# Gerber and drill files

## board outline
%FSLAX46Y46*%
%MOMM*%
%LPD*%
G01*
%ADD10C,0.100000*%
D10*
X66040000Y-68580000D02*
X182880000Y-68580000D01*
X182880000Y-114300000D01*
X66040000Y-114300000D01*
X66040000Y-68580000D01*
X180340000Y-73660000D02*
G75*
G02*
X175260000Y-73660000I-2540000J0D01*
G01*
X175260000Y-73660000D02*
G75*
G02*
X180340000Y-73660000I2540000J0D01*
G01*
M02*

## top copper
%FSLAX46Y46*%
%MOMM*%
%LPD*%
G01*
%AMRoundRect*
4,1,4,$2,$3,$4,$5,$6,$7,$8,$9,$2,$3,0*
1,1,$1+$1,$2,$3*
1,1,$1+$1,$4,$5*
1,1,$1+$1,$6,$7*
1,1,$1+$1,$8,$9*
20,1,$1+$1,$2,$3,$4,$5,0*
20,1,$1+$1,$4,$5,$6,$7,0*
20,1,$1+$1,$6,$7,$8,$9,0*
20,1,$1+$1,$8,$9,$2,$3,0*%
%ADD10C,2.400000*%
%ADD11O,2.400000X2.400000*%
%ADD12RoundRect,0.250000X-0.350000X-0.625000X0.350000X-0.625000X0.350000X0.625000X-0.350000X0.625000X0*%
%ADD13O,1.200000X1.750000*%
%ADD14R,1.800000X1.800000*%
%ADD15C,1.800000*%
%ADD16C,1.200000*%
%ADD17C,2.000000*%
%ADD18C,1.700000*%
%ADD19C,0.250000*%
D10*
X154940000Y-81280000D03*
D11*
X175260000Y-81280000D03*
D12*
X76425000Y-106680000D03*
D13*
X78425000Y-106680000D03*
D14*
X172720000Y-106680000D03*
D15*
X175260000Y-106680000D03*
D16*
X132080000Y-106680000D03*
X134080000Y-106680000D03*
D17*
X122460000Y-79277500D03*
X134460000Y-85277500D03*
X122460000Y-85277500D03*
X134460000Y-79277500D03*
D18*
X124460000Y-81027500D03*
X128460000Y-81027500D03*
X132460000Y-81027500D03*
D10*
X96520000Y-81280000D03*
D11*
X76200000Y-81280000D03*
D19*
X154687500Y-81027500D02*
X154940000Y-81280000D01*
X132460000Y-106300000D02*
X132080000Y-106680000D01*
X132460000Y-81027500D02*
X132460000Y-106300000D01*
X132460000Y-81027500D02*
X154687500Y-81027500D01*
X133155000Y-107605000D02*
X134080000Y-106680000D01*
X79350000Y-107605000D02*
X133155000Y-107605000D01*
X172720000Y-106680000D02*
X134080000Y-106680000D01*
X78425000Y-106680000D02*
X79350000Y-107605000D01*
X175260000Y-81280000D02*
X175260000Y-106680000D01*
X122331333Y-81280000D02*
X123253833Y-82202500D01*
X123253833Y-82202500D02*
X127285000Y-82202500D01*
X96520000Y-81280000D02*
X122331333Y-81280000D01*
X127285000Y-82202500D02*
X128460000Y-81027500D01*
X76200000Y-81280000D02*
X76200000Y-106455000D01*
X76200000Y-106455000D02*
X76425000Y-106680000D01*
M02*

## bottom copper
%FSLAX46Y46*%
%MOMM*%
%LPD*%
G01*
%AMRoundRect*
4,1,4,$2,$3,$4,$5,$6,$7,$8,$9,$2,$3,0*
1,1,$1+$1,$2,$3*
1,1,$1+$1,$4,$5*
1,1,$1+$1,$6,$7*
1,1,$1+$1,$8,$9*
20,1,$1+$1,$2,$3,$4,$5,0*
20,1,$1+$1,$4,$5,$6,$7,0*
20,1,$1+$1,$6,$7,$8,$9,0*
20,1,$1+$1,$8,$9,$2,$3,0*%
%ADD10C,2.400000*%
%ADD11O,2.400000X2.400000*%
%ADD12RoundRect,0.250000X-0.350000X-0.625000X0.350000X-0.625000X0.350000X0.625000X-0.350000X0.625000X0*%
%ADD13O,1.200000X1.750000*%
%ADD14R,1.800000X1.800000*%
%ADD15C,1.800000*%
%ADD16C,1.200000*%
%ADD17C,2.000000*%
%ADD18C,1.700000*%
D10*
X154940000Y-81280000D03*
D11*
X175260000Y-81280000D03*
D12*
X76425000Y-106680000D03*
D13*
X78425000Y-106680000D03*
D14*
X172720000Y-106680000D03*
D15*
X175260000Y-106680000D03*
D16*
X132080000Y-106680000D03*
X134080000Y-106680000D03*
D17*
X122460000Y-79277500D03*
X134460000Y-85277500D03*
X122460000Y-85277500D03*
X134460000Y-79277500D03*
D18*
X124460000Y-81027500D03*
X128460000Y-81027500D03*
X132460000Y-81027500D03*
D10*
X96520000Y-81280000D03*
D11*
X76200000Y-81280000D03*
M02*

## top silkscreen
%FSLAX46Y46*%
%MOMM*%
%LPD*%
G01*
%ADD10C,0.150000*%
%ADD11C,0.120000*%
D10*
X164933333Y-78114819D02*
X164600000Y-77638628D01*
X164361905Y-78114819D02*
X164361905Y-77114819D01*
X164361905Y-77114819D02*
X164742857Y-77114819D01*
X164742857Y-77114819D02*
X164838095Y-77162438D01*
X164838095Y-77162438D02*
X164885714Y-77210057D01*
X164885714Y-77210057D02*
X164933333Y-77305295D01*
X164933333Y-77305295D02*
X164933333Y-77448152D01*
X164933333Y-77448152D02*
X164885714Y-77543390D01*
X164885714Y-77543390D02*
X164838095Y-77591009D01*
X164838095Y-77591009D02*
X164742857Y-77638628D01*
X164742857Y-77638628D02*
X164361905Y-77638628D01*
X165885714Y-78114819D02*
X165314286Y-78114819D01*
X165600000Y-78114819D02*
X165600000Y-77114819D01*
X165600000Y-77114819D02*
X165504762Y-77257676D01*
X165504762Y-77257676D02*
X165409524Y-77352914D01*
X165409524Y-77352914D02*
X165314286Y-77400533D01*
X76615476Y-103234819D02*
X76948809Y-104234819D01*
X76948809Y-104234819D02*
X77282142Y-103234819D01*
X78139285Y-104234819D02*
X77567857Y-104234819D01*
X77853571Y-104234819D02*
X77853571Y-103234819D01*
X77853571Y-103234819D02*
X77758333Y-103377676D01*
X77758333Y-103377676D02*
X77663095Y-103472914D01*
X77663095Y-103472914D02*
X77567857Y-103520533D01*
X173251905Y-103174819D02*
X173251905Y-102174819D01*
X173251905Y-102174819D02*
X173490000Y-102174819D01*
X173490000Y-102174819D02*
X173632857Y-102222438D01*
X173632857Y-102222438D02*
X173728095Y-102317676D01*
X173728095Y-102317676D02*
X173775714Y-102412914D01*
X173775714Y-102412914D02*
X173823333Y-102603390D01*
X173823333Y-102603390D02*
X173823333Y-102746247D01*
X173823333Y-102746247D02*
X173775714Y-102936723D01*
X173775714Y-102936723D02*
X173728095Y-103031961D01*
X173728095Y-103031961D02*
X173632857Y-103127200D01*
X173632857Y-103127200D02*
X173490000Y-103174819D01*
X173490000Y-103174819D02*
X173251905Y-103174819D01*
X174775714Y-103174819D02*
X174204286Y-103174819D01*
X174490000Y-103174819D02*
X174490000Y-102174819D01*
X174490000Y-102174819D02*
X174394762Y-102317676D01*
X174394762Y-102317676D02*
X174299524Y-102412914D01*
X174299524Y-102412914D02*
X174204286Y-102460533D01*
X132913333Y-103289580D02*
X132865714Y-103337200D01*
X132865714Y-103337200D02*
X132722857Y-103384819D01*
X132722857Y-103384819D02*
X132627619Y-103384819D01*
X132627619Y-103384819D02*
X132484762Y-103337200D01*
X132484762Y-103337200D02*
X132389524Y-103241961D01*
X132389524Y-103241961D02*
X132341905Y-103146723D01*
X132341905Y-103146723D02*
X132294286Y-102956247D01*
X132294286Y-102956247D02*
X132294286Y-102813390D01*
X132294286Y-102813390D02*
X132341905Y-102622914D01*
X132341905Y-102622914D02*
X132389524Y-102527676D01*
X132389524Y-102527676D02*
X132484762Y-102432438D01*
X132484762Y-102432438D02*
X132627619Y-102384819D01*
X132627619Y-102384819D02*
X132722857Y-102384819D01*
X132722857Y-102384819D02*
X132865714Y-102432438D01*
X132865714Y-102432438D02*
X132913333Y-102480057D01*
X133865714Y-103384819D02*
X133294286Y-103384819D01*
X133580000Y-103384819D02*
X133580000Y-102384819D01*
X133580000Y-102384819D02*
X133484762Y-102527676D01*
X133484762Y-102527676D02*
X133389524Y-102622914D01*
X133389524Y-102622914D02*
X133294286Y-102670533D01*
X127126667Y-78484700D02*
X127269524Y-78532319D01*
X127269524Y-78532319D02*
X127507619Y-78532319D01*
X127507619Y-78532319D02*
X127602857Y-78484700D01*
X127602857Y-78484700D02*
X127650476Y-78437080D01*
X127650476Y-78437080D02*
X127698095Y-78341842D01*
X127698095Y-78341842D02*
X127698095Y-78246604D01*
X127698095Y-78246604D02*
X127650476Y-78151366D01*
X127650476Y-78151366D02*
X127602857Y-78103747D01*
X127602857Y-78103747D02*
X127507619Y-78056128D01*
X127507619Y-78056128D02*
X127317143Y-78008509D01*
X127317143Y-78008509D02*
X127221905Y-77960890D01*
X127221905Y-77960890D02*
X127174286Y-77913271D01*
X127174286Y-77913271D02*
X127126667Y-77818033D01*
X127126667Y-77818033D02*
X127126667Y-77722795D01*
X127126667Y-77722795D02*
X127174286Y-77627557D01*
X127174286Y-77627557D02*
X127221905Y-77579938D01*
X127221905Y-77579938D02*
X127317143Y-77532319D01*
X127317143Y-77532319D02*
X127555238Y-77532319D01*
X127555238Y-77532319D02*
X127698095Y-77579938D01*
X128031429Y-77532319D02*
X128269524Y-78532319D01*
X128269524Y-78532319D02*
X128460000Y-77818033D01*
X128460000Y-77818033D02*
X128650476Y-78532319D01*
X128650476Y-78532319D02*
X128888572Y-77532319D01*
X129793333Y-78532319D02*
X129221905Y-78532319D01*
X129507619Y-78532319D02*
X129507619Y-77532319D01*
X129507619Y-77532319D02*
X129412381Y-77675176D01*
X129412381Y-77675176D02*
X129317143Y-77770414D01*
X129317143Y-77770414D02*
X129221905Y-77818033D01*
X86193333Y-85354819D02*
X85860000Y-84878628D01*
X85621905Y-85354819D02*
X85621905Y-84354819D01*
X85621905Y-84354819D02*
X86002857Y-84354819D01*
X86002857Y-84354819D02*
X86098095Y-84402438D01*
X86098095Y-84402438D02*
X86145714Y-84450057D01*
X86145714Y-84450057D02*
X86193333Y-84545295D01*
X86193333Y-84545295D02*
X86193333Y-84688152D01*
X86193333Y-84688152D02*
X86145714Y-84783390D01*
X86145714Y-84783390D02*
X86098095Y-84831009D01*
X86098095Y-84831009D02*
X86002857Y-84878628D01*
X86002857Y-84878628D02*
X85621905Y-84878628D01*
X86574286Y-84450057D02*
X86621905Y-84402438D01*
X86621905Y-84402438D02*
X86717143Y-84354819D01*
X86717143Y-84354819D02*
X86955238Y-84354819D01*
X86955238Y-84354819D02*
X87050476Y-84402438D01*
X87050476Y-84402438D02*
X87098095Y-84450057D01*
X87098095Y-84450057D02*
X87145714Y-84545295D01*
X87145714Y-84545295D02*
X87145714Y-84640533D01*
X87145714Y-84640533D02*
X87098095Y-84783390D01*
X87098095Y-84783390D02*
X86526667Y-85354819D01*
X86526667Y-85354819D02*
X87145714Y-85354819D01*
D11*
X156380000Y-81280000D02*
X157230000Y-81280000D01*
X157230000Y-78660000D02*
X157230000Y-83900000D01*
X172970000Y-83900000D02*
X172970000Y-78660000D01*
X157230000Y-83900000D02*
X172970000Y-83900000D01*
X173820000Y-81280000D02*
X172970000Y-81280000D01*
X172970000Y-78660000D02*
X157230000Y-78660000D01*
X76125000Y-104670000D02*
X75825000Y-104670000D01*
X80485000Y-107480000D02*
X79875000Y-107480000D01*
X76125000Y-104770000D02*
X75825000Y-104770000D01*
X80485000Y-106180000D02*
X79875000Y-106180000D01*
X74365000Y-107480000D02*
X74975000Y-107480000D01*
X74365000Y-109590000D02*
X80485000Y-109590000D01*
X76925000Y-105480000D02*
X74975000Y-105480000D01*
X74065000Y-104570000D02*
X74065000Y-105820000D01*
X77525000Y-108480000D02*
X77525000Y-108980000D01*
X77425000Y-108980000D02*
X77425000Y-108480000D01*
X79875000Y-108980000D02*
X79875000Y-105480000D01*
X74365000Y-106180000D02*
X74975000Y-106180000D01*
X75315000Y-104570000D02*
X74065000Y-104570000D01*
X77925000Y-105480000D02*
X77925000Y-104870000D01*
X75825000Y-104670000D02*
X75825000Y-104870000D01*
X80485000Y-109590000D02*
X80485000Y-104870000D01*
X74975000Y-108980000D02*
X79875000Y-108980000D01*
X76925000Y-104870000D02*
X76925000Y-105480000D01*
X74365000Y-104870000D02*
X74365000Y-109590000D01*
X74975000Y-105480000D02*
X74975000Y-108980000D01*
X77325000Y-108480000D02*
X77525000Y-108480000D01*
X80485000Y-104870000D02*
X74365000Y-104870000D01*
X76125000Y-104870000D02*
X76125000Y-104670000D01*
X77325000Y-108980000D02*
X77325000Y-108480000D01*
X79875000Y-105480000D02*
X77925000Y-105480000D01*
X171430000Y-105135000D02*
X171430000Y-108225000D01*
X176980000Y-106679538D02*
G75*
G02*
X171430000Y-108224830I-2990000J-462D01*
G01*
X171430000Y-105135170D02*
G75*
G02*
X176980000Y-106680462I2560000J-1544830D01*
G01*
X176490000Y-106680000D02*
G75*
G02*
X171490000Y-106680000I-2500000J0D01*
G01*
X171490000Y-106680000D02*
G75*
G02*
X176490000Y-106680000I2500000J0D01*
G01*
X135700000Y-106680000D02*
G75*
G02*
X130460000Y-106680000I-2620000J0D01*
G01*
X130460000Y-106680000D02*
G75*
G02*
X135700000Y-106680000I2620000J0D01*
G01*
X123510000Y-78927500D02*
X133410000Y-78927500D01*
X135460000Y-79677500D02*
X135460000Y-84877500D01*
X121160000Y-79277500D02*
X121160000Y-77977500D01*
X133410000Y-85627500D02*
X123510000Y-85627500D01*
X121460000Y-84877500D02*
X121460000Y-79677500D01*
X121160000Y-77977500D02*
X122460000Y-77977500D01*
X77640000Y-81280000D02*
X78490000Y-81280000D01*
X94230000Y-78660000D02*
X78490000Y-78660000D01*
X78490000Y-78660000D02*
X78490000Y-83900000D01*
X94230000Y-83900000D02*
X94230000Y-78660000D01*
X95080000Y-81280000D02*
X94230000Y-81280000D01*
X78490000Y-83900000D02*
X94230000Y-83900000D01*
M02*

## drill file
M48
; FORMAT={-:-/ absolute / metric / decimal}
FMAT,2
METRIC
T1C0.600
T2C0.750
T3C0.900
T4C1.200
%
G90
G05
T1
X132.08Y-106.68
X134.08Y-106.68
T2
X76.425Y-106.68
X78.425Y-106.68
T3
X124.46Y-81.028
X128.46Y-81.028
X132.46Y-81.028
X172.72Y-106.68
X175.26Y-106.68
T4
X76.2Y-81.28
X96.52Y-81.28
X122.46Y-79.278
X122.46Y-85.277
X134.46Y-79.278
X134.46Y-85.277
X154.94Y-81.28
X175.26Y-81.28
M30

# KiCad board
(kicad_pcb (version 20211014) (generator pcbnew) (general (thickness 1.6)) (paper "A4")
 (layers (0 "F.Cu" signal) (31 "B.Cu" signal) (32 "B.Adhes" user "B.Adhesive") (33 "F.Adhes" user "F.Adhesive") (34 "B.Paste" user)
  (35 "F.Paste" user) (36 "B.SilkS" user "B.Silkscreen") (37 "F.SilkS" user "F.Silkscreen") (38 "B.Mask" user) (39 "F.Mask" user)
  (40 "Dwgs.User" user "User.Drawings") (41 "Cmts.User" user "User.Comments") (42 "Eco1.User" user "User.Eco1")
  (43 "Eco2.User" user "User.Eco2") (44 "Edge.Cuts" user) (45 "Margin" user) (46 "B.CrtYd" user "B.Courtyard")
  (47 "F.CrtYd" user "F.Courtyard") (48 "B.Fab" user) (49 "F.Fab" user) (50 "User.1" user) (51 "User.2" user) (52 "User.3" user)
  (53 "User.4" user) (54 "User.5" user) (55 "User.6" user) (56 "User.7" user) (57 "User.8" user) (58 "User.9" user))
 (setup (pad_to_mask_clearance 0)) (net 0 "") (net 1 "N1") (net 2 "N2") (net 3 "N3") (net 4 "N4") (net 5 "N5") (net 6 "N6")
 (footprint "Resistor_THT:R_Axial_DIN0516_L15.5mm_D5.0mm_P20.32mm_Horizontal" (layer "F.Cu") (at 154.94 81.28)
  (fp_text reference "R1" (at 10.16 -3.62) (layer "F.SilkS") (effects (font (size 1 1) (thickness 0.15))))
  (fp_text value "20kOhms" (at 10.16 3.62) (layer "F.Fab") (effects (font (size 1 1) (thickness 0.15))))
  (fp_line (start 1.44 0) (end 2.29 0) (layer "F.SilkS") (width 0.12))
  (fp_line (start 2.29 -2.62) (end 2.29 2.62) (layer "F.SilkS") (width 0.12))
  (fp_line (start 18.03 2.62) (end 18.03 -2.62) (layer "F.SilkS") (width 0.12))
  (fp_line (start 2.29 2.62) (end 18.03 2.62) (layer "F.SilkS") (width 0.12))
  (fp_line (start 18.88 0) (end 18.03 0) (layer "F.SilkS") (width 0.12))
  (fp_line (start 18.03 -2.62) (end 2.29 -2.62) (layer "F.SilkS") (width 0.12))
  (pad "1" thru_hole circle (at 0 0) (size 2.4 2.4) (drill 1.2) (layers *.Cu *.Mask) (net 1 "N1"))
  (pad "2" thru_hole oval (at 20.32 0) (size 2.4 2.4) (drill 1.2) (layers *.Cu *.Mask) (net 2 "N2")))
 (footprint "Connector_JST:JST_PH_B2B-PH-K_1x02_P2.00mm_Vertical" (layer "F.Cu") (at 76.425 106.68)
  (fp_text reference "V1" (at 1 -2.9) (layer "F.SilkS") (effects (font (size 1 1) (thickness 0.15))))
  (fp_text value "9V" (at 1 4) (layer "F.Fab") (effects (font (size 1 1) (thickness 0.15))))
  (fp_line (start -0.3 -2.01) (end -0.6 -2.01) (layer "F.SilkS") (width 0.12))
  (fp_line (start 4.06 0.8) (end 3.45 0.8) (layer "F.SilkS") (width 0.12))
  (fp_line (start -0.3 -1.91) (end -0.6 -1.91) (layer "F.SilkS") (width 0.12))
  (fp_line (start 4.06 -0.5) (end 3.45 -0.5) (layer "F.SilkS") (width 0.12))
  (fp_line (start -2.06 0.8) (end -1.45 0.8) (layer "F.SilkS") (width 0.12))
  (fp_line (start -2.06 2.91) (end 4.06 2.91) (layer "F.SilkS") (width 0.12))
  (fp_line (start 0.5 -1.2) (end -1.45 -1.2) (layer "F.SilkS") (width 0.12))
  (fp_line (start -2.36 -2.11) (end -2.36 -0.86) (layer "F.SilkS") (width 0.12))
  (fp_line (start 1.1 1.8) (end 1.1 2.3) (layer "F.SilkS") (width 0.12))
  (fp_line (start 1 2.3) (end 1 1.8) (layer "F.SilkS") (width 0.12))
  (fp_line (start 3.45 2.3) (end 3.45 -1.2) (layer "F.SilkS") (width 0.12))
  (fp_line (start -2.06 -0.5) (end -1.45 -0.5) (layer "F.SilkS") (width 0.12))
  (fp_line (start -1.11 -2.11) (end -2.36 -2.11) (layer "F.SilkS") (width 0.12))
  (fp_line (start 1.5 -1.2) (end 1.5 -1.81) (layer "F.SilkS") (width 0.12))
  (fp_line (start -0.6 -2.01) (end -0.6 -1.81) (layer "F.SilkS") (width 0.12))
  (fp_line (start 4.06 2.91) (end 4.06 -1.81) (layer "F.SilkS") (width 0.12))
  (fp_line (start -1.45 2.3) (end 3.45 2.3) (layer "F.SilkS") (width 0.12))
  (fp_line (start 0.5 -1.81) (end 0.5 -1.2) (layer "F.SilkS") (width 0.12))
  (fp_line (start -2.06 -1.81) (end -2.06 2.91) (layer "F.SilkS") (width 0.12))
  (fp_line (start -1.45 -1.2) (end -1.45 2.3) (layer "F.SilkS") (width 0.12))
  (fp_line (start 0.9 1.8) (end 1.1 1.8) (layer "F.SilkS") (width 0.12))
  (fp_line (start 4.06 -1.81) (end -2.06 -1.81) (layer "F.SilkS") (width 0.12))
  (fp_line (start -0.3 -1.81) (end -0.3 -2.01) (layer "F.SilkS") (width 0.12))
  (fp_line (start 0.9 2.3) (end 0.9 1.8) (layer "F.SilkS") (width 0.12))
  (fp_line (start 3.45 -1.2) (end 1.5 -1.2) (layer "F.SilkS") (width 0.12))
  (pad "1" thru_hole roundrect (at 0 0) (size 1.2 1.75) (drill 0.75) (layers *.Cu *.Mask) (roundrect_rratio 0.208333) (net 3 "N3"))
  (pad "2" thru_hole oval (at 2 0) (size 1.2 1.75) (drill 0.75) (layers *.Cu *.Mask) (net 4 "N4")))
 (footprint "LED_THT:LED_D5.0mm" (layer "F.Cu") (at 172.72 106.68)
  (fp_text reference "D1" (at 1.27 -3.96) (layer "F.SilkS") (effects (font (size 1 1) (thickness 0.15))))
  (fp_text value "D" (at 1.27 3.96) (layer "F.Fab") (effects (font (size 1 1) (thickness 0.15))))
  (fp_line (start -1.29 -1.545) (end -1.29 1.545) (layer "F.SilkS") (width 0.12))
  (fp_arc (start 4.26 -0.000462) (mid 2.072002 2.880433) (end -1.29 1.54483) (layer "F.SilkS") (width 0.12))
  (fp_arc (start -1.29 -1.54483) (mid 2.072002 -2.880433) (end 4.26 0.000462) (layer "F.SilkS") (width 0.12))
  (fp_circle (center 1.27 0) (end 3.77 0) (layer "F.SilkS") (width 0.12) (fill none))
  (pad "1" thru_hole rect (at 0 0) (size 1.8 1.8) (drill 0.9) (layers *.Cu *.Mask) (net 4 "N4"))
  (pad "2" thru_hole circle (at 2.54 0) (size 1.8 1.8) (drill 0.9) (layers *.Cu *.Mask) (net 2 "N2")))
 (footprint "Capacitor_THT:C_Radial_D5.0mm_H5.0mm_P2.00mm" (layer "F.Cu") (at 132.08 106.68)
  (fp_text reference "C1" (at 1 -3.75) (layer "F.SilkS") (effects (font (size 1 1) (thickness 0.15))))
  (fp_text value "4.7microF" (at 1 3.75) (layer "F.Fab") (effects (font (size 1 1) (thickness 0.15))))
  (fp_circle (center 1 0) (end 3.62 0) (layer "F.SilkS") (width 0.12) (fill none))
  (pad "1" thru_hole circle (at 0 0) (size 1.2 1.2) (drill 0.6) (layers *.Cu *.Mask) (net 1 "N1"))
  (pad "2" thru_hole circle (at 2 0) (size 1.2 1.2) (drill 0.6) (layers *.Cu *.Mask) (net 4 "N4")))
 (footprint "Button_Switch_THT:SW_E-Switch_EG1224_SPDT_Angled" (layer "F.Cu") (at 124.46 81.0275)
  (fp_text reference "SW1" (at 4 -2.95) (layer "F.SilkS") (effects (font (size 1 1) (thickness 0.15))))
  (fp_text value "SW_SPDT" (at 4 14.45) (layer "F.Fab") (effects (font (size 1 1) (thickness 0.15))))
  (fp_line (start -0.95 -2.1) (end 8.95 -2.1) (layer "F.SilkS") (width 0.12))
  (fp_line (start 11 -1.35) (end 11 3.85) (layer "F.SilkS") (width 0.12))
  (fp_line (start -3.3 -1.75) (end -3.3 -3.05) (layer "F.SilkS") (width 0.12))
  (fp_line (start 8.95 4.6) (end -0.95 4.6) (layer "F.SilkS") (width 0.12))
  (fp_line (start -3 3.85) (end -3 -1.35) (layer "F.SilkS") (width 0.12))
  (fp_line (start -3.3 -3.05) (end -2 -3.05) (layer "F.SilkS") (width 0.12))
  (pad "" thru_hole circle (at -2 -1.75) (size 2 2) (drill 1.2) (layers *.Cu *.Mask))
  (pad "" thru_hole circle (at 10 4.25) (size 2 2) (drill 1.2) (layers *.Cu *.Mask))
  (pad "" thru_hole circle (at -2 4.25) (size 2 2) (drill 1.2) (layers *.Cu *.Mask))
  (pad "" thru_hole circle (at 10 -1.75) (size 2 2) (drill 1.2) (layers *.Cu *.Mask))
  (pad "1" thru_hole circle (at 0 0) (size 1.7 1.7) (drill 0.9) (layers *.Cu *.Mask) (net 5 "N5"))
  (pad "2" thru_hole circle (at 4 0) (size 1.7 1.7) (drill 0.9) (layers *.Cu *.Mask) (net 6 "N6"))
  (pad "3" thru_hole circle (at 8 0) (size 1.7 1.7) (drill 0.9) (layers *.Cu *.Mask) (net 1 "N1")))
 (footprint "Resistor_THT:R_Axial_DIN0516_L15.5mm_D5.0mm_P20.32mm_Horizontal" (layer "F.Cu") (at 96.52 81.28 180)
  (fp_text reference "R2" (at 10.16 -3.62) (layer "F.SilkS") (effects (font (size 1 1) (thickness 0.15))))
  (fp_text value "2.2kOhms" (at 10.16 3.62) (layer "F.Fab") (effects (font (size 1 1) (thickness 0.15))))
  (fp_line (start 18.88 0) (end 18.03 0) (layer "F.SilkS") (width 0.12))
  (fp_line (start 2.29 2.62) (end 18.03 2.62) (layer "F.SilkS") (width 0.12))
  (fp_line (start 18.03 2.62) (end 18.03 -2.62) (layer "F.SilkS") (width 0.12))
  (fp_line (start 2.29 -2.62) (end 2.29 2.62) (layer "F.SilkS") (width 0.12))
  (fp_line (start 1.44 0) (end 2.29 0) (layer "F.SilkS") (width 0.12))
  (fp_line (start 18.03 -2.62) (end 2.29 -2.62) (layer "F.SilkS") (width 0.12))
  (pad "1" thru_hole circle (at 0 0 180) (size 2.4 2.4) (drill 1.2) (layers *.Cu *.Mask) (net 6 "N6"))
  (pad "2" thru_hole oval (at 20.32 0 180) (size 2.4 2.4) (drill 1.2) (layers *.Cu *.Mask) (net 3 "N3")))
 (gr_rect (start 66.04 68.58) (end 182.88 114.3) (layer "Edge.Cuts") (width 0.1) (fill none))
 (gr_circle (center 177.8 73.66) (end 175.26 73.66) (layer "Edge.Cuts") (width 0.1) (fill none))
 (segment (start 154.6875 81.0275) (end 154.94 81.28) (width 0.25) (layer "F.Cu") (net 1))
 (segment (start 132.46 106.3) (end 132.08 106.68) (width 0.25) (layer "F.Cu") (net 1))
 (segment (start 132.46 81.0275) (end 132.46 106.3) (width 0.25) (layer "F.Cu") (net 1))
 (segment (start 132.46 81.0275) (end 154.6875 81.0275) (width 0.25) (layer "F.Cu") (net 1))
 (segment (start 133.155 107.605) (end 134.08 106.68) (width 0.25) (layer "F.Cu") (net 4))
 (segment (start 79.35 107.605) (end 133.155 107.605) (width 0.25) (layer "F.Cu") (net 4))
 (segment (start 172.72 106.68) (end 134.08 106.68) (width 0.25) (layer "F.Cu") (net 4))
 (segment (start 78.425 106.68) (end 79.35 107.605) (width 0.25) (layer "F.Cu") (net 4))
 (segment (start 175.26 81.28) (end 175.26 106.68) (width 0.25) (layer "F.Cu") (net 2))
 (segment (start 122.331333 81.28) (end 123.253833 82.2025) (width 0.25) (layer "F.Cu") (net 6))
 (segment (start 123.253833 82.2025) (end 127.285 82.2025) (width 0.25) (layer "F.Cu") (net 6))
 (segment (start 96.52 81.28) (end 122.331333 81.28) (width 0.25) (layer "F.Cu") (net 6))
 (segment (start 127.285 82.2025) (end 128.46 81.0275) (width 0.25) (layer "F.Cu") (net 6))
 (segment (start 76.2 81.28) (end 76.2 106.455) (width 0.25) (layer "F.Cu") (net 3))
 (segment (start 76.2 106.455) (end 76.425 106.68) (width 0.25) (layer "F.Cu") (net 3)))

